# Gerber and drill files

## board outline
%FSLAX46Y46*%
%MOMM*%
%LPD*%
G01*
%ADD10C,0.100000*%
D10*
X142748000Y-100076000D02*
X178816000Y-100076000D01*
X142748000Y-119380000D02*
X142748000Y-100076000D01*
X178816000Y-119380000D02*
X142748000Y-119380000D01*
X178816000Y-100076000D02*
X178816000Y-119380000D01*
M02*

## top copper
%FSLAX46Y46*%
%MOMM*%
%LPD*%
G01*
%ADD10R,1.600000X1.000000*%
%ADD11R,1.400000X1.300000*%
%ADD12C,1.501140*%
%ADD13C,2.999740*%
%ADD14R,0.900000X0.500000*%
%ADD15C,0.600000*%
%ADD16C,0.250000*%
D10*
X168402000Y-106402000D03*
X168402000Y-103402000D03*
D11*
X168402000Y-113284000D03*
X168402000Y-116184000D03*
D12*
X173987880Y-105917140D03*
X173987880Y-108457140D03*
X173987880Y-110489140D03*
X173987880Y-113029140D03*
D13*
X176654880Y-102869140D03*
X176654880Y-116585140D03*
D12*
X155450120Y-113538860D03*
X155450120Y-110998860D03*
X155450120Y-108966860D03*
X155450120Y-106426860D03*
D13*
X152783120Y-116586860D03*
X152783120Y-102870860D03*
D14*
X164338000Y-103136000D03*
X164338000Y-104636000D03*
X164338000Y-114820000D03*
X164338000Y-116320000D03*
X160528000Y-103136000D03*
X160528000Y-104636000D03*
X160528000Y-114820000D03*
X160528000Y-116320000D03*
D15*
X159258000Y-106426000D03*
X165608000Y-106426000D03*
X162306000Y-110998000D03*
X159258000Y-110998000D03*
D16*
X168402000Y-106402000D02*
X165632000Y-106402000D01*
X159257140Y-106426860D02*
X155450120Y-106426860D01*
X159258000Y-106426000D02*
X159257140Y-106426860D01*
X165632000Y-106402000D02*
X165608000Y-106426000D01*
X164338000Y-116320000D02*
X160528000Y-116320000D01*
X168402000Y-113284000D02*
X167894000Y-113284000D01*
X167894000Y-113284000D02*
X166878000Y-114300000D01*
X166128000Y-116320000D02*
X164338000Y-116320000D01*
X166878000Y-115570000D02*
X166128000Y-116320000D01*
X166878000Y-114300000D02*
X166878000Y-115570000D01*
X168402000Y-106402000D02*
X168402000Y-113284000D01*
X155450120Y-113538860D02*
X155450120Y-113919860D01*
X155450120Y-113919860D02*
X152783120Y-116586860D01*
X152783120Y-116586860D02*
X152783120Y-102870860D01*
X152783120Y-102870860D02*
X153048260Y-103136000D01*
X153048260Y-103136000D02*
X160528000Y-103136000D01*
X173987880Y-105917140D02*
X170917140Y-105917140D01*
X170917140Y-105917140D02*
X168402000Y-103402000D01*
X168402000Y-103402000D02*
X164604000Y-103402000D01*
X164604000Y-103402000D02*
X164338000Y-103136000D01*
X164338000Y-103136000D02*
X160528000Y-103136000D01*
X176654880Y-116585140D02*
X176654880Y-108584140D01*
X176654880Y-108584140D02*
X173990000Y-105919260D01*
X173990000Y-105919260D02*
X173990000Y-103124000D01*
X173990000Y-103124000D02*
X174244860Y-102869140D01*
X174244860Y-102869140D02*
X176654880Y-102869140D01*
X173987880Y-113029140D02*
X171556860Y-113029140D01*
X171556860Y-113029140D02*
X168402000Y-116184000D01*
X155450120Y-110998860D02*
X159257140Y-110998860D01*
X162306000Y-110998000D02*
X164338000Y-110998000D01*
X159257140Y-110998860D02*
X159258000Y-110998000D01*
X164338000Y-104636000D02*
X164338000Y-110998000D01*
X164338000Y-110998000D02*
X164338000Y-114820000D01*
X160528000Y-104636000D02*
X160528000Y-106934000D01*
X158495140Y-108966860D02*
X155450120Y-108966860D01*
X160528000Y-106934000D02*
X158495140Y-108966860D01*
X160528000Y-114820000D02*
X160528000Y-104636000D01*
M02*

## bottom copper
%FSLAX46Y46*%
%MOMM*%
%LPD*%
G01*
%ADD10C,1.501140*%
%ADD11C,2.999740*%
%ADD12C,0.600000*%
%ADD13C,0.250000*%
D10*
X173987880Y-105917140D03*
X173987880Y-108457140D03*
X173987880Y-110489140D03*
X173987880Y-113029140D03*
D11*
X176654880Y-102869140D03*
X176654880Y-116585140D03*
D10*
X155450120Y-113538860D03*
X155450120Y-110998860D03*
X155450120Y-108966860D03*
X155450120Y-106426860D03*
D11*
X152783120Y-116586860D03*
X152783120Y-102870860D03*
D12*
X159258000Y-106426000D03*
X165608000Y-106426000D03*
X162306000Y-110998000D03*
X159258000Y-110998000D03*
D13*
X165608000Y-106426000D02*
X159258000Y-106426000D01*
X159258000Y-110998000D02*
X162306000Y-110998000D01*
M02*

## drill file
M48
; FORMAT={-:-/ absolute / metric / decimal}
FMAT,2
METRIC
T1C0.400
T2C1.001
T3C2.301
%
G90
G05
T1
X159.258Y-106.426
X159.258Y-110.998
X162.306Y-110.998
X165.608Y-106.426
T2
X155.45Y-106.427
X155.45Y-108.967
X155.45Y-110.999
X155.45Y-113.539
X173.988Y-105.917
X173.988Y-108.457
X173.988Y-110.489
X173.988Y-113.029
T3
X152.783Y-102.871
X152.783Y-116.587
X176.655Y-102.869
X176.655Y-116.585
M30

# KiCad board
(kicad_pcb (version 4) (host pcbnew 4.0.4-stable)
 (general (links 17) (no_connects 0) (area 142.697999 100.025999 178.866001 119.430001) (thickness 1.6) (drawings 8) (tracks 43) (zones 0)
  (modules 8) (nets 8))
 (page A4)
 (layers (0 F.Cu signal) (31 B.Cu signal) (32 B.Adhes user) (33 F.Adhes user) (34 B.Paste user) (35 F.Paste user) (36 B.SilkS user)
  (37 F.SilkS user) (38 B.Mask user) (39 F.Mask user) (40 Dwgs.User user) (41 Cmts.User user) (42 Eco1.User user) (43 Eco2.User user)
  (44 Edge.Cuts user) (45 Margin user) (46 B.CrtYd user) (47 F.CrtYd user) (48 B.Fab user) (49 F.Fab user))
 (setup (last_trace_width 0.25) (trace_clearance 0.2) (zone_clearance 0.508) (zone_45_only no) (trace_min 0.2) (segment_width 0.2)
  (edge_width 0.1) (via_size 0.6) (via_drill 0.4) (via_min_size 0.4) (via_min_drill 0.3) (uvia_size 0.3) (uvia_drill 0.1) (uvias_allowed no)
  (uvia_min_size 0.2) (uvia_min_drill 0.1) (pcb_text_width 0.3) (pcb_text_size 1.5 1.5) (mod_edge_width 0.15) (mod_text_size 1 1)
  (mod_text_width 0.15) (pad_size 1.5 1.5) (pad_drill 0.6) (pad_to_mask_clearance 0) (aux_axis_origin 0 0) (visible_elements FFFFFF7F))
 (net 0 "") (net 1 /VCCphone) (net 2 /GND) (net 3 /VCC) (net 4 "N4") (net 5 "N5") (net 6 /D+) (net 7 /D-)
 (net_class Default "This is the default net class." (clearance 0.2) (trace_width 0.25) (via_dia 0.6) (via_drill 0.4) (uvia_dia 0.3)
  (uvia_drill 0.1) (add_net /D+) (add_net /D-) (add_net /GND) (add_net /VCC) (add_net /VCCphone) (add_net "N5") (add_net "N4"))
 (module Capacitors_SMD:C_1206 (layer F.Cu) (at 168.402 104.902 90)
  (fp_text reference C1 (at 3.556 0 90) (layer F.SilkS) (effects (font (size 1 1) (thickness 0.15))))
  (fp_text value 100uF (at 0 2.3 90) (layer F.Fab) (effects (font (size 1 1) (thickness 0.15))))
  (pad 1 smd rect (at -1.5 0 90) (size 1 1.6) (layers F.Cu F.Paste F.Mask) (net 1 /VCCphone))
  (pad 2 smd rect (at 1.5 0 90) (size 1 1.6) (layers F.Cu F.Paste F.Mask) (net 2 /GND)))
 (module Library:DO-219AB (layer F.Cu) (at 170.942 113.284 270)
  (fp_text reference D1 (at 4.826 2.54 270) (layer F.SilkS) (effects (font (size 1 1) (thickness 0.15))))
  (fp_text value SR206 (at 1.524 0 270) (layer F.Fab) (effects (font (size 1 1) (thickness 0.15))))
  (pad 1 smd rect (at 0 2.54 270) (size 1.3 1.4) (layers F.Cu F.Paste F.Mask) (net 1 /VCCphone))
  (pad 2 smd rect (at 2.9 2.54 270) (size 1.3 1.4) (layers F.Cu F.Paste F.Mask) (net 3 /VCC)))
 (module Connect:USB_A (layer F.Cu) (at 173.99 113.03 90)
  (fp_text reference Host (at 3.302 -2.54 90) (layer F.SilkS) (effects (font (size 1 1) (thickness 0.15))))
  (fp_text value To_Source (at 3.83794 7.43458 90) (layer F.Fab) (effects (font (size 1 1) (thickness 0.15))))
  (pad 4 thru_hole circle (at 7.11286 -0.00212) (size 1.50114 1.50114) (drill 1.00076) (layers *.Cu *.Mask F.SilkS) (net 2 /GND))
  (pad 3 thru_hole circle (at 4.57286 -0.00212) (size 1.50114 1.50114) (drill 1.00076) (layers *.Cu *.Mask F.SilkS) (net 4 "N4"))
  (pad 2 thru_hole circle (at 2.54086 -0.00212) (size 1.50114 1.50114) (drill 1.00076) (layers *.Cu *.Mask F.SilkS) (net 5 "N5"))
  (pad 1 thru_hole circle (at 0.00086 -0.00212) (size 1.50114 1.50114) (drill 1.00076) (layers *.Cu *.Mask F.SilkS) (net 3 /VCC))
  (pad 5 thru_hole circle (at 10.16086 2.66488) (size 2.99974 2.99974) (drill 2.30124) (layers *.Cu *.Mask F.SilkS) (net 2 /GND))
  (pad 5 thru_hole circle (at -3.55514 2.66488) (size 2.99974 2.99974) (drill 2.30124) (layers *.Cu *.Mask F.SilkS) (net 2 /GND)))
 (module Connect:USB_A (layer F.Cu) (at 155.448 106.426 270)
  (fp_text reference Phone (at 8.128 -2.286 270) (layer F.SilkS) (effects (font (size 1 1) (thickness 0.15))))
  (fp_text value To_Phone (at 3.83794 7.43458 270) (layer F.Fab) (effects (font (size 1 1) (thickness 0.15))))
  (pad 4 thru_hole circle (at 7.11286 -0.00212 180) (size 1.50114 1.50114) (drill 1.00076) (layers *.Cu *.Mask F.SilkS) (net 2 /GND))
  (pad 3 thru_hole circle (at 4.57286 -0.00212 180) (size 1.50114 1.50114) (drill 1.00076) (layers *.Cu *.Mask F.SilkS) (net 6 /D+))
  (pad 2 thru_hole circle (at 2.54086 -0.00212 180) (size 1.50114 1.50114) (drill 1.00076) (layers *.Cu *.Mask F.SilkS) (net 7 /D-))
  (pad 1 thru_hole circle (at 0.00086 -0.00212 180) (size 1.50114 1.50114) (drill 1.00076) (layers *.Cu *.Mask F.SilkS) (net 1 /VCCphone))
  (pad 5 thru_hole circle (at 10.16086 2.66488 180) (size 2.99974 2.99974) (drill 2.30124) (layers *.Cu *.Mask F.SilkS) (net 2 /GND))
  (pad 5 thru_hole circle (at -3.55514 2.66488 180) (size 2.99974 2.99974) (drill 2.30124) (layers *.Cu *.Mask F.SilkS) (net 2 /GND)))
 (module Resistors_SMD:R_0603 (layer F.Cu) (at 164.338 103.886 270)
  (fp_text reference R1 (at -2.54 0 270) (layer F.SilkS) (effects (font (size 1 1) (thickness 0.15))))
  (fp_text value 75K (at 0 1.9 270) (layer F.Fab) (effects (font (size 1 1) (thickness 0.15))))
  (pad 1 smd rect (at -0.75 0 270) (size 0.5 0.9) (layers F.Cu F.Paste F.Mask) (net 2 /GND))
  (pad 2 smd rect (at 0.75 0 270) (size 0.5 0.9) (layers F.Cu F.Paste F.Mask) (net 6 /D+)))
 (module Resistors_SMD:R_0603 (layer F.Cu) (at 164.338 115.57 270)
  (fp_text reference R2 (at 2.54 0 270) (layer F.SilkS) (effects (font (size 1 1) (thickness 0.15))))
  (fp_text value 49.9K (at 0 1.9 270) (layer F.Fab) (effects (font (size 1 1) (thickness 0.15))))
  (pad 1 smd rect (at -0.75 0 270) (size 0.5 0.9) (layers F.Cu F.Paste F.Mask) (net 6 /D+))
  (pad 2 smd rect (at 0.75 0 270) (size 0.5 0.9) (layers F.Cu F.Paste F.Mask) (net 1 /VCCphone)))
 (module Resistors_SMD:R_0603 (layer F.Cu) (at 160.528 103.886 270)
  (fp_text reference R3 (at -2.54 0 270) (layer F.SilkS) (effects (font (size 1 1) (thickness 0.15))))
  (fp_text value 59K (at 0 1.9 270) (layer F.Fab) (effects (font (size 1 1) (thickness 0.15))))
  (pad 1 smd rect (at -0.75 0 270) (size 0.5 0.9) (layers F.Cu F.Paste F.Mask) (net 2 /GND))
  (pad 2 smd rect (at 0.75 0 270) (size 0.5 0.9) (layers F.Cu F.Paste F.Mask) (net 7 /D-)))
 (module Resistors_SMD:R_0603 (layer F.Cu) (at 160.528 115.57 270)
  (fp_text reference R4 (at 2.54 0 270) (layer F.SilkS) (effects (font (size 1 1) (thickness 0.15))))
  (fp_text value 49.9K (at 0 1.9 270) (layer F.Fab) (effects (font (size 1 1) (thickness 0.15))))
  (pad 1 smd rect (at -0.75 0 270) (size 0.5 0.9) (layers F.Cu F.Paste F.Mask) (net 7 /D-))
  (pad 2 smd rect (at 0.75 0 270) (size 0.5 0.9) (layers F.Cu F.Paste F.Mask) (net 1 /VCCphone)))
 (gr_line (start 142.748 100.076) (end 178.816 100.076) (angle 90) (layer Edge.Cuts) (width 0.1))
 (gr_line (start 142.748 119.38) (end 142.748 100.076) (angle 90) (layer Edge.Cuts) (width 0.1))
 (gr_line (start 178.816 119.38) (end 142.748 119.38) (angle 90) (layer Edge.Cuts) (width 0.1))
 (gr_line (start 178.816 100.076) (end 178.816 119.38) (angle 90) (layer Edge.Cuts) (width 0.1))
 (segment (start 168.402 106.402) (end 165.632 106.402) (width 0.25) (layer F.Cu) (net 1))
 (segment (start 159.25714 106.42686) (end 155.45012 106.42686) (width 0.25) (layer F.Cu) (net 1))
 (segment (start 159.258 106.426) (end 159.25714 106.42686) (width 0.25) (layer F.Cu) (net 1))
 (via (at 159.258 106.426) (size 0.6) (drill 0.4) (layers F.Cu B.Cu) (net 1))
 (segment (start 165.608 106.426) (end 159.258 106.426) (width 0.25) (layer B.Cu) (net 1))
 (via (at 165.608 106.426) (size 0.6) (drill 0.4) (layers F.Cu B.Cu) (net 1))
 (segment (start 165.632 106.402) (end 165.608 106.426) (width 0.25) (layer F.Cu) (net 1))
 (segment (start 164.338 116.32) (end 160.528 116.32) (width 0.25) (layer F.Cu) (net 1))
 (segment (start 168.402 113.284) (end 167.894 113.284) (width 0.25) (layer F.Cu) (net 1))
 (segment (start 167.894 113.284) (end 166.878 114.3) (width 0.25) (layer F.Cu) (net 1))
 (segment (start 166.128 116.32) (end 164.338 116.32) (width 0.25) (layer F.Cu) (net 1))
 (segment (start 166.878 115.57) (end 166.128 116.32) (width 0.25) (layer F.Cu) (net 1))
 (segment (start 166.878 114.3) (end 166.878 115.57) (width 0.25) (layer F.Cu) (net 1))
 (segment (start 168.402 106.402) (end 168.402 113.284) (width 0.25) (layer F.Cu) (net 1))
 (segment (start 155.45012 113.53886) (end 155.45012 113.91986) (width 0.25) (layer F.Cu) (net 2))
 (segment (start 155.45012 113.91986) (end 152.78312 116.58686) (width 0.25) (layer F.Cu) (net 2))
 (segment (start 152.78312 116.58686) (end 152.78312 102.87086) (width 0.25) (layer F.Cu) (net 2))
 (segment (start 152.78312 102.87086) (end 153.04826 103.136) (width 0.25) (layer F.Cu) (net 2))
 (segment (start 153.04826 103.136) (end 160.528 103.136) (width 0.25) (layer F.Cu) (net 2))
 (segment (start 173.98788 105.91714) (end 170.91714 105.91714) (width 0.25) (layer F.Cu) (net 2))
 (segment (start 170.91714 105.91714) (end 168.402 103.402) (width 0.25) (layer F.Cu) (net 2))
 (segment (start 168.402 103.402) (end 164.604 103.402) (width 0.25) (layer F.Cu) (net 2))
 (segment (start 164.604 103.402) (end 164.338 103.136) (width 0.25) (layer F.Cu) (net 2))
 (segment (start 164.338 103.136) (end 160.528 103.136) (width 0.25) (layer F.Cu) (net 2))
 (segment (start 176.65488 116.58514) (end 176.65488 108.58414) (width 0.25) (layer F.Cu) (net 2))
 (segment (start 176.65488 108.58414) (end 173.99 105.91926) (width 0.25) (layer F.Cu) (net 2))
 (segment (start 173.99 105.91926) (end 173.99 103.124) (width 0.25) (layer F.Cu) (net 2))
 (segment (start 173.99 103.124) (end 174.24486 102.86914) (width 0.25) (layer F.Cu) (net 2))
 (segment (start 174.24486 102.86914) (end 176.65488 102.86914) (width 0.25) (layer F.Cu) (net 2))
 (segment (start 173.98788 113.02914) (end 171.55686 113.02914) (width 0.25) (layer F.Cu) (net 3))
 (segment (start 171.55686 113.02914) (end 168.402 116.184) (width 0.25) (layer F.Cu) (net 3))
 (segment (start 155.45012 110.99886) (end 159.25714 110.99886) (width 0.25) (layer F.Cu) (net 6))
 (segment (start 162.306 110.998) (end 164.338 110.998) (width 0.25) (layer F.Cu) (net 6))
 (via (at 162.306 110.998) (size 0.6) (drill 0.4) (layers F.Cu B.Cu) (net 6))
 (segment (start 159.258 110.998) (end 162.306 110.998) (width 0.25) (layer B.Cu) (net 6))
 (via (at 159.258 110.998) (size 0.6) (drill 0.4) (layers F.Cu B.Cu) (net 6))
 (segment (start 159.25714 110.99886) (end 159.258 110.998) (width 0.25) (layer F.Cu) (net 6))
 (segment (start 164.338 104.636) (end 164.338 110.998) (width 0.25) (layer F.Cu) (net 6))
 (segment (start 164.338 110.998) (end 164.338 114.82) (width 0.25) (layer F.Cu) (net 6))
 (segment (start 160.528 104.636) (end 160.528 106.934) (width 0.25) (layer F.Cu) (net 7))
 (segment (start 158.49514 108.96686) (end 155.45012 108.96686) (width 0.25) (layer F.Cu) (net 7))
 (segment (start 160.528 106.934) (end 158.49514 108.96686) (width 0.25) (layer F.Cu) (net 7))
 (segment (start 160.528 114.82) (end 160.528 104.636) (width 0.25) (layer F.Cu) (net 7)))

